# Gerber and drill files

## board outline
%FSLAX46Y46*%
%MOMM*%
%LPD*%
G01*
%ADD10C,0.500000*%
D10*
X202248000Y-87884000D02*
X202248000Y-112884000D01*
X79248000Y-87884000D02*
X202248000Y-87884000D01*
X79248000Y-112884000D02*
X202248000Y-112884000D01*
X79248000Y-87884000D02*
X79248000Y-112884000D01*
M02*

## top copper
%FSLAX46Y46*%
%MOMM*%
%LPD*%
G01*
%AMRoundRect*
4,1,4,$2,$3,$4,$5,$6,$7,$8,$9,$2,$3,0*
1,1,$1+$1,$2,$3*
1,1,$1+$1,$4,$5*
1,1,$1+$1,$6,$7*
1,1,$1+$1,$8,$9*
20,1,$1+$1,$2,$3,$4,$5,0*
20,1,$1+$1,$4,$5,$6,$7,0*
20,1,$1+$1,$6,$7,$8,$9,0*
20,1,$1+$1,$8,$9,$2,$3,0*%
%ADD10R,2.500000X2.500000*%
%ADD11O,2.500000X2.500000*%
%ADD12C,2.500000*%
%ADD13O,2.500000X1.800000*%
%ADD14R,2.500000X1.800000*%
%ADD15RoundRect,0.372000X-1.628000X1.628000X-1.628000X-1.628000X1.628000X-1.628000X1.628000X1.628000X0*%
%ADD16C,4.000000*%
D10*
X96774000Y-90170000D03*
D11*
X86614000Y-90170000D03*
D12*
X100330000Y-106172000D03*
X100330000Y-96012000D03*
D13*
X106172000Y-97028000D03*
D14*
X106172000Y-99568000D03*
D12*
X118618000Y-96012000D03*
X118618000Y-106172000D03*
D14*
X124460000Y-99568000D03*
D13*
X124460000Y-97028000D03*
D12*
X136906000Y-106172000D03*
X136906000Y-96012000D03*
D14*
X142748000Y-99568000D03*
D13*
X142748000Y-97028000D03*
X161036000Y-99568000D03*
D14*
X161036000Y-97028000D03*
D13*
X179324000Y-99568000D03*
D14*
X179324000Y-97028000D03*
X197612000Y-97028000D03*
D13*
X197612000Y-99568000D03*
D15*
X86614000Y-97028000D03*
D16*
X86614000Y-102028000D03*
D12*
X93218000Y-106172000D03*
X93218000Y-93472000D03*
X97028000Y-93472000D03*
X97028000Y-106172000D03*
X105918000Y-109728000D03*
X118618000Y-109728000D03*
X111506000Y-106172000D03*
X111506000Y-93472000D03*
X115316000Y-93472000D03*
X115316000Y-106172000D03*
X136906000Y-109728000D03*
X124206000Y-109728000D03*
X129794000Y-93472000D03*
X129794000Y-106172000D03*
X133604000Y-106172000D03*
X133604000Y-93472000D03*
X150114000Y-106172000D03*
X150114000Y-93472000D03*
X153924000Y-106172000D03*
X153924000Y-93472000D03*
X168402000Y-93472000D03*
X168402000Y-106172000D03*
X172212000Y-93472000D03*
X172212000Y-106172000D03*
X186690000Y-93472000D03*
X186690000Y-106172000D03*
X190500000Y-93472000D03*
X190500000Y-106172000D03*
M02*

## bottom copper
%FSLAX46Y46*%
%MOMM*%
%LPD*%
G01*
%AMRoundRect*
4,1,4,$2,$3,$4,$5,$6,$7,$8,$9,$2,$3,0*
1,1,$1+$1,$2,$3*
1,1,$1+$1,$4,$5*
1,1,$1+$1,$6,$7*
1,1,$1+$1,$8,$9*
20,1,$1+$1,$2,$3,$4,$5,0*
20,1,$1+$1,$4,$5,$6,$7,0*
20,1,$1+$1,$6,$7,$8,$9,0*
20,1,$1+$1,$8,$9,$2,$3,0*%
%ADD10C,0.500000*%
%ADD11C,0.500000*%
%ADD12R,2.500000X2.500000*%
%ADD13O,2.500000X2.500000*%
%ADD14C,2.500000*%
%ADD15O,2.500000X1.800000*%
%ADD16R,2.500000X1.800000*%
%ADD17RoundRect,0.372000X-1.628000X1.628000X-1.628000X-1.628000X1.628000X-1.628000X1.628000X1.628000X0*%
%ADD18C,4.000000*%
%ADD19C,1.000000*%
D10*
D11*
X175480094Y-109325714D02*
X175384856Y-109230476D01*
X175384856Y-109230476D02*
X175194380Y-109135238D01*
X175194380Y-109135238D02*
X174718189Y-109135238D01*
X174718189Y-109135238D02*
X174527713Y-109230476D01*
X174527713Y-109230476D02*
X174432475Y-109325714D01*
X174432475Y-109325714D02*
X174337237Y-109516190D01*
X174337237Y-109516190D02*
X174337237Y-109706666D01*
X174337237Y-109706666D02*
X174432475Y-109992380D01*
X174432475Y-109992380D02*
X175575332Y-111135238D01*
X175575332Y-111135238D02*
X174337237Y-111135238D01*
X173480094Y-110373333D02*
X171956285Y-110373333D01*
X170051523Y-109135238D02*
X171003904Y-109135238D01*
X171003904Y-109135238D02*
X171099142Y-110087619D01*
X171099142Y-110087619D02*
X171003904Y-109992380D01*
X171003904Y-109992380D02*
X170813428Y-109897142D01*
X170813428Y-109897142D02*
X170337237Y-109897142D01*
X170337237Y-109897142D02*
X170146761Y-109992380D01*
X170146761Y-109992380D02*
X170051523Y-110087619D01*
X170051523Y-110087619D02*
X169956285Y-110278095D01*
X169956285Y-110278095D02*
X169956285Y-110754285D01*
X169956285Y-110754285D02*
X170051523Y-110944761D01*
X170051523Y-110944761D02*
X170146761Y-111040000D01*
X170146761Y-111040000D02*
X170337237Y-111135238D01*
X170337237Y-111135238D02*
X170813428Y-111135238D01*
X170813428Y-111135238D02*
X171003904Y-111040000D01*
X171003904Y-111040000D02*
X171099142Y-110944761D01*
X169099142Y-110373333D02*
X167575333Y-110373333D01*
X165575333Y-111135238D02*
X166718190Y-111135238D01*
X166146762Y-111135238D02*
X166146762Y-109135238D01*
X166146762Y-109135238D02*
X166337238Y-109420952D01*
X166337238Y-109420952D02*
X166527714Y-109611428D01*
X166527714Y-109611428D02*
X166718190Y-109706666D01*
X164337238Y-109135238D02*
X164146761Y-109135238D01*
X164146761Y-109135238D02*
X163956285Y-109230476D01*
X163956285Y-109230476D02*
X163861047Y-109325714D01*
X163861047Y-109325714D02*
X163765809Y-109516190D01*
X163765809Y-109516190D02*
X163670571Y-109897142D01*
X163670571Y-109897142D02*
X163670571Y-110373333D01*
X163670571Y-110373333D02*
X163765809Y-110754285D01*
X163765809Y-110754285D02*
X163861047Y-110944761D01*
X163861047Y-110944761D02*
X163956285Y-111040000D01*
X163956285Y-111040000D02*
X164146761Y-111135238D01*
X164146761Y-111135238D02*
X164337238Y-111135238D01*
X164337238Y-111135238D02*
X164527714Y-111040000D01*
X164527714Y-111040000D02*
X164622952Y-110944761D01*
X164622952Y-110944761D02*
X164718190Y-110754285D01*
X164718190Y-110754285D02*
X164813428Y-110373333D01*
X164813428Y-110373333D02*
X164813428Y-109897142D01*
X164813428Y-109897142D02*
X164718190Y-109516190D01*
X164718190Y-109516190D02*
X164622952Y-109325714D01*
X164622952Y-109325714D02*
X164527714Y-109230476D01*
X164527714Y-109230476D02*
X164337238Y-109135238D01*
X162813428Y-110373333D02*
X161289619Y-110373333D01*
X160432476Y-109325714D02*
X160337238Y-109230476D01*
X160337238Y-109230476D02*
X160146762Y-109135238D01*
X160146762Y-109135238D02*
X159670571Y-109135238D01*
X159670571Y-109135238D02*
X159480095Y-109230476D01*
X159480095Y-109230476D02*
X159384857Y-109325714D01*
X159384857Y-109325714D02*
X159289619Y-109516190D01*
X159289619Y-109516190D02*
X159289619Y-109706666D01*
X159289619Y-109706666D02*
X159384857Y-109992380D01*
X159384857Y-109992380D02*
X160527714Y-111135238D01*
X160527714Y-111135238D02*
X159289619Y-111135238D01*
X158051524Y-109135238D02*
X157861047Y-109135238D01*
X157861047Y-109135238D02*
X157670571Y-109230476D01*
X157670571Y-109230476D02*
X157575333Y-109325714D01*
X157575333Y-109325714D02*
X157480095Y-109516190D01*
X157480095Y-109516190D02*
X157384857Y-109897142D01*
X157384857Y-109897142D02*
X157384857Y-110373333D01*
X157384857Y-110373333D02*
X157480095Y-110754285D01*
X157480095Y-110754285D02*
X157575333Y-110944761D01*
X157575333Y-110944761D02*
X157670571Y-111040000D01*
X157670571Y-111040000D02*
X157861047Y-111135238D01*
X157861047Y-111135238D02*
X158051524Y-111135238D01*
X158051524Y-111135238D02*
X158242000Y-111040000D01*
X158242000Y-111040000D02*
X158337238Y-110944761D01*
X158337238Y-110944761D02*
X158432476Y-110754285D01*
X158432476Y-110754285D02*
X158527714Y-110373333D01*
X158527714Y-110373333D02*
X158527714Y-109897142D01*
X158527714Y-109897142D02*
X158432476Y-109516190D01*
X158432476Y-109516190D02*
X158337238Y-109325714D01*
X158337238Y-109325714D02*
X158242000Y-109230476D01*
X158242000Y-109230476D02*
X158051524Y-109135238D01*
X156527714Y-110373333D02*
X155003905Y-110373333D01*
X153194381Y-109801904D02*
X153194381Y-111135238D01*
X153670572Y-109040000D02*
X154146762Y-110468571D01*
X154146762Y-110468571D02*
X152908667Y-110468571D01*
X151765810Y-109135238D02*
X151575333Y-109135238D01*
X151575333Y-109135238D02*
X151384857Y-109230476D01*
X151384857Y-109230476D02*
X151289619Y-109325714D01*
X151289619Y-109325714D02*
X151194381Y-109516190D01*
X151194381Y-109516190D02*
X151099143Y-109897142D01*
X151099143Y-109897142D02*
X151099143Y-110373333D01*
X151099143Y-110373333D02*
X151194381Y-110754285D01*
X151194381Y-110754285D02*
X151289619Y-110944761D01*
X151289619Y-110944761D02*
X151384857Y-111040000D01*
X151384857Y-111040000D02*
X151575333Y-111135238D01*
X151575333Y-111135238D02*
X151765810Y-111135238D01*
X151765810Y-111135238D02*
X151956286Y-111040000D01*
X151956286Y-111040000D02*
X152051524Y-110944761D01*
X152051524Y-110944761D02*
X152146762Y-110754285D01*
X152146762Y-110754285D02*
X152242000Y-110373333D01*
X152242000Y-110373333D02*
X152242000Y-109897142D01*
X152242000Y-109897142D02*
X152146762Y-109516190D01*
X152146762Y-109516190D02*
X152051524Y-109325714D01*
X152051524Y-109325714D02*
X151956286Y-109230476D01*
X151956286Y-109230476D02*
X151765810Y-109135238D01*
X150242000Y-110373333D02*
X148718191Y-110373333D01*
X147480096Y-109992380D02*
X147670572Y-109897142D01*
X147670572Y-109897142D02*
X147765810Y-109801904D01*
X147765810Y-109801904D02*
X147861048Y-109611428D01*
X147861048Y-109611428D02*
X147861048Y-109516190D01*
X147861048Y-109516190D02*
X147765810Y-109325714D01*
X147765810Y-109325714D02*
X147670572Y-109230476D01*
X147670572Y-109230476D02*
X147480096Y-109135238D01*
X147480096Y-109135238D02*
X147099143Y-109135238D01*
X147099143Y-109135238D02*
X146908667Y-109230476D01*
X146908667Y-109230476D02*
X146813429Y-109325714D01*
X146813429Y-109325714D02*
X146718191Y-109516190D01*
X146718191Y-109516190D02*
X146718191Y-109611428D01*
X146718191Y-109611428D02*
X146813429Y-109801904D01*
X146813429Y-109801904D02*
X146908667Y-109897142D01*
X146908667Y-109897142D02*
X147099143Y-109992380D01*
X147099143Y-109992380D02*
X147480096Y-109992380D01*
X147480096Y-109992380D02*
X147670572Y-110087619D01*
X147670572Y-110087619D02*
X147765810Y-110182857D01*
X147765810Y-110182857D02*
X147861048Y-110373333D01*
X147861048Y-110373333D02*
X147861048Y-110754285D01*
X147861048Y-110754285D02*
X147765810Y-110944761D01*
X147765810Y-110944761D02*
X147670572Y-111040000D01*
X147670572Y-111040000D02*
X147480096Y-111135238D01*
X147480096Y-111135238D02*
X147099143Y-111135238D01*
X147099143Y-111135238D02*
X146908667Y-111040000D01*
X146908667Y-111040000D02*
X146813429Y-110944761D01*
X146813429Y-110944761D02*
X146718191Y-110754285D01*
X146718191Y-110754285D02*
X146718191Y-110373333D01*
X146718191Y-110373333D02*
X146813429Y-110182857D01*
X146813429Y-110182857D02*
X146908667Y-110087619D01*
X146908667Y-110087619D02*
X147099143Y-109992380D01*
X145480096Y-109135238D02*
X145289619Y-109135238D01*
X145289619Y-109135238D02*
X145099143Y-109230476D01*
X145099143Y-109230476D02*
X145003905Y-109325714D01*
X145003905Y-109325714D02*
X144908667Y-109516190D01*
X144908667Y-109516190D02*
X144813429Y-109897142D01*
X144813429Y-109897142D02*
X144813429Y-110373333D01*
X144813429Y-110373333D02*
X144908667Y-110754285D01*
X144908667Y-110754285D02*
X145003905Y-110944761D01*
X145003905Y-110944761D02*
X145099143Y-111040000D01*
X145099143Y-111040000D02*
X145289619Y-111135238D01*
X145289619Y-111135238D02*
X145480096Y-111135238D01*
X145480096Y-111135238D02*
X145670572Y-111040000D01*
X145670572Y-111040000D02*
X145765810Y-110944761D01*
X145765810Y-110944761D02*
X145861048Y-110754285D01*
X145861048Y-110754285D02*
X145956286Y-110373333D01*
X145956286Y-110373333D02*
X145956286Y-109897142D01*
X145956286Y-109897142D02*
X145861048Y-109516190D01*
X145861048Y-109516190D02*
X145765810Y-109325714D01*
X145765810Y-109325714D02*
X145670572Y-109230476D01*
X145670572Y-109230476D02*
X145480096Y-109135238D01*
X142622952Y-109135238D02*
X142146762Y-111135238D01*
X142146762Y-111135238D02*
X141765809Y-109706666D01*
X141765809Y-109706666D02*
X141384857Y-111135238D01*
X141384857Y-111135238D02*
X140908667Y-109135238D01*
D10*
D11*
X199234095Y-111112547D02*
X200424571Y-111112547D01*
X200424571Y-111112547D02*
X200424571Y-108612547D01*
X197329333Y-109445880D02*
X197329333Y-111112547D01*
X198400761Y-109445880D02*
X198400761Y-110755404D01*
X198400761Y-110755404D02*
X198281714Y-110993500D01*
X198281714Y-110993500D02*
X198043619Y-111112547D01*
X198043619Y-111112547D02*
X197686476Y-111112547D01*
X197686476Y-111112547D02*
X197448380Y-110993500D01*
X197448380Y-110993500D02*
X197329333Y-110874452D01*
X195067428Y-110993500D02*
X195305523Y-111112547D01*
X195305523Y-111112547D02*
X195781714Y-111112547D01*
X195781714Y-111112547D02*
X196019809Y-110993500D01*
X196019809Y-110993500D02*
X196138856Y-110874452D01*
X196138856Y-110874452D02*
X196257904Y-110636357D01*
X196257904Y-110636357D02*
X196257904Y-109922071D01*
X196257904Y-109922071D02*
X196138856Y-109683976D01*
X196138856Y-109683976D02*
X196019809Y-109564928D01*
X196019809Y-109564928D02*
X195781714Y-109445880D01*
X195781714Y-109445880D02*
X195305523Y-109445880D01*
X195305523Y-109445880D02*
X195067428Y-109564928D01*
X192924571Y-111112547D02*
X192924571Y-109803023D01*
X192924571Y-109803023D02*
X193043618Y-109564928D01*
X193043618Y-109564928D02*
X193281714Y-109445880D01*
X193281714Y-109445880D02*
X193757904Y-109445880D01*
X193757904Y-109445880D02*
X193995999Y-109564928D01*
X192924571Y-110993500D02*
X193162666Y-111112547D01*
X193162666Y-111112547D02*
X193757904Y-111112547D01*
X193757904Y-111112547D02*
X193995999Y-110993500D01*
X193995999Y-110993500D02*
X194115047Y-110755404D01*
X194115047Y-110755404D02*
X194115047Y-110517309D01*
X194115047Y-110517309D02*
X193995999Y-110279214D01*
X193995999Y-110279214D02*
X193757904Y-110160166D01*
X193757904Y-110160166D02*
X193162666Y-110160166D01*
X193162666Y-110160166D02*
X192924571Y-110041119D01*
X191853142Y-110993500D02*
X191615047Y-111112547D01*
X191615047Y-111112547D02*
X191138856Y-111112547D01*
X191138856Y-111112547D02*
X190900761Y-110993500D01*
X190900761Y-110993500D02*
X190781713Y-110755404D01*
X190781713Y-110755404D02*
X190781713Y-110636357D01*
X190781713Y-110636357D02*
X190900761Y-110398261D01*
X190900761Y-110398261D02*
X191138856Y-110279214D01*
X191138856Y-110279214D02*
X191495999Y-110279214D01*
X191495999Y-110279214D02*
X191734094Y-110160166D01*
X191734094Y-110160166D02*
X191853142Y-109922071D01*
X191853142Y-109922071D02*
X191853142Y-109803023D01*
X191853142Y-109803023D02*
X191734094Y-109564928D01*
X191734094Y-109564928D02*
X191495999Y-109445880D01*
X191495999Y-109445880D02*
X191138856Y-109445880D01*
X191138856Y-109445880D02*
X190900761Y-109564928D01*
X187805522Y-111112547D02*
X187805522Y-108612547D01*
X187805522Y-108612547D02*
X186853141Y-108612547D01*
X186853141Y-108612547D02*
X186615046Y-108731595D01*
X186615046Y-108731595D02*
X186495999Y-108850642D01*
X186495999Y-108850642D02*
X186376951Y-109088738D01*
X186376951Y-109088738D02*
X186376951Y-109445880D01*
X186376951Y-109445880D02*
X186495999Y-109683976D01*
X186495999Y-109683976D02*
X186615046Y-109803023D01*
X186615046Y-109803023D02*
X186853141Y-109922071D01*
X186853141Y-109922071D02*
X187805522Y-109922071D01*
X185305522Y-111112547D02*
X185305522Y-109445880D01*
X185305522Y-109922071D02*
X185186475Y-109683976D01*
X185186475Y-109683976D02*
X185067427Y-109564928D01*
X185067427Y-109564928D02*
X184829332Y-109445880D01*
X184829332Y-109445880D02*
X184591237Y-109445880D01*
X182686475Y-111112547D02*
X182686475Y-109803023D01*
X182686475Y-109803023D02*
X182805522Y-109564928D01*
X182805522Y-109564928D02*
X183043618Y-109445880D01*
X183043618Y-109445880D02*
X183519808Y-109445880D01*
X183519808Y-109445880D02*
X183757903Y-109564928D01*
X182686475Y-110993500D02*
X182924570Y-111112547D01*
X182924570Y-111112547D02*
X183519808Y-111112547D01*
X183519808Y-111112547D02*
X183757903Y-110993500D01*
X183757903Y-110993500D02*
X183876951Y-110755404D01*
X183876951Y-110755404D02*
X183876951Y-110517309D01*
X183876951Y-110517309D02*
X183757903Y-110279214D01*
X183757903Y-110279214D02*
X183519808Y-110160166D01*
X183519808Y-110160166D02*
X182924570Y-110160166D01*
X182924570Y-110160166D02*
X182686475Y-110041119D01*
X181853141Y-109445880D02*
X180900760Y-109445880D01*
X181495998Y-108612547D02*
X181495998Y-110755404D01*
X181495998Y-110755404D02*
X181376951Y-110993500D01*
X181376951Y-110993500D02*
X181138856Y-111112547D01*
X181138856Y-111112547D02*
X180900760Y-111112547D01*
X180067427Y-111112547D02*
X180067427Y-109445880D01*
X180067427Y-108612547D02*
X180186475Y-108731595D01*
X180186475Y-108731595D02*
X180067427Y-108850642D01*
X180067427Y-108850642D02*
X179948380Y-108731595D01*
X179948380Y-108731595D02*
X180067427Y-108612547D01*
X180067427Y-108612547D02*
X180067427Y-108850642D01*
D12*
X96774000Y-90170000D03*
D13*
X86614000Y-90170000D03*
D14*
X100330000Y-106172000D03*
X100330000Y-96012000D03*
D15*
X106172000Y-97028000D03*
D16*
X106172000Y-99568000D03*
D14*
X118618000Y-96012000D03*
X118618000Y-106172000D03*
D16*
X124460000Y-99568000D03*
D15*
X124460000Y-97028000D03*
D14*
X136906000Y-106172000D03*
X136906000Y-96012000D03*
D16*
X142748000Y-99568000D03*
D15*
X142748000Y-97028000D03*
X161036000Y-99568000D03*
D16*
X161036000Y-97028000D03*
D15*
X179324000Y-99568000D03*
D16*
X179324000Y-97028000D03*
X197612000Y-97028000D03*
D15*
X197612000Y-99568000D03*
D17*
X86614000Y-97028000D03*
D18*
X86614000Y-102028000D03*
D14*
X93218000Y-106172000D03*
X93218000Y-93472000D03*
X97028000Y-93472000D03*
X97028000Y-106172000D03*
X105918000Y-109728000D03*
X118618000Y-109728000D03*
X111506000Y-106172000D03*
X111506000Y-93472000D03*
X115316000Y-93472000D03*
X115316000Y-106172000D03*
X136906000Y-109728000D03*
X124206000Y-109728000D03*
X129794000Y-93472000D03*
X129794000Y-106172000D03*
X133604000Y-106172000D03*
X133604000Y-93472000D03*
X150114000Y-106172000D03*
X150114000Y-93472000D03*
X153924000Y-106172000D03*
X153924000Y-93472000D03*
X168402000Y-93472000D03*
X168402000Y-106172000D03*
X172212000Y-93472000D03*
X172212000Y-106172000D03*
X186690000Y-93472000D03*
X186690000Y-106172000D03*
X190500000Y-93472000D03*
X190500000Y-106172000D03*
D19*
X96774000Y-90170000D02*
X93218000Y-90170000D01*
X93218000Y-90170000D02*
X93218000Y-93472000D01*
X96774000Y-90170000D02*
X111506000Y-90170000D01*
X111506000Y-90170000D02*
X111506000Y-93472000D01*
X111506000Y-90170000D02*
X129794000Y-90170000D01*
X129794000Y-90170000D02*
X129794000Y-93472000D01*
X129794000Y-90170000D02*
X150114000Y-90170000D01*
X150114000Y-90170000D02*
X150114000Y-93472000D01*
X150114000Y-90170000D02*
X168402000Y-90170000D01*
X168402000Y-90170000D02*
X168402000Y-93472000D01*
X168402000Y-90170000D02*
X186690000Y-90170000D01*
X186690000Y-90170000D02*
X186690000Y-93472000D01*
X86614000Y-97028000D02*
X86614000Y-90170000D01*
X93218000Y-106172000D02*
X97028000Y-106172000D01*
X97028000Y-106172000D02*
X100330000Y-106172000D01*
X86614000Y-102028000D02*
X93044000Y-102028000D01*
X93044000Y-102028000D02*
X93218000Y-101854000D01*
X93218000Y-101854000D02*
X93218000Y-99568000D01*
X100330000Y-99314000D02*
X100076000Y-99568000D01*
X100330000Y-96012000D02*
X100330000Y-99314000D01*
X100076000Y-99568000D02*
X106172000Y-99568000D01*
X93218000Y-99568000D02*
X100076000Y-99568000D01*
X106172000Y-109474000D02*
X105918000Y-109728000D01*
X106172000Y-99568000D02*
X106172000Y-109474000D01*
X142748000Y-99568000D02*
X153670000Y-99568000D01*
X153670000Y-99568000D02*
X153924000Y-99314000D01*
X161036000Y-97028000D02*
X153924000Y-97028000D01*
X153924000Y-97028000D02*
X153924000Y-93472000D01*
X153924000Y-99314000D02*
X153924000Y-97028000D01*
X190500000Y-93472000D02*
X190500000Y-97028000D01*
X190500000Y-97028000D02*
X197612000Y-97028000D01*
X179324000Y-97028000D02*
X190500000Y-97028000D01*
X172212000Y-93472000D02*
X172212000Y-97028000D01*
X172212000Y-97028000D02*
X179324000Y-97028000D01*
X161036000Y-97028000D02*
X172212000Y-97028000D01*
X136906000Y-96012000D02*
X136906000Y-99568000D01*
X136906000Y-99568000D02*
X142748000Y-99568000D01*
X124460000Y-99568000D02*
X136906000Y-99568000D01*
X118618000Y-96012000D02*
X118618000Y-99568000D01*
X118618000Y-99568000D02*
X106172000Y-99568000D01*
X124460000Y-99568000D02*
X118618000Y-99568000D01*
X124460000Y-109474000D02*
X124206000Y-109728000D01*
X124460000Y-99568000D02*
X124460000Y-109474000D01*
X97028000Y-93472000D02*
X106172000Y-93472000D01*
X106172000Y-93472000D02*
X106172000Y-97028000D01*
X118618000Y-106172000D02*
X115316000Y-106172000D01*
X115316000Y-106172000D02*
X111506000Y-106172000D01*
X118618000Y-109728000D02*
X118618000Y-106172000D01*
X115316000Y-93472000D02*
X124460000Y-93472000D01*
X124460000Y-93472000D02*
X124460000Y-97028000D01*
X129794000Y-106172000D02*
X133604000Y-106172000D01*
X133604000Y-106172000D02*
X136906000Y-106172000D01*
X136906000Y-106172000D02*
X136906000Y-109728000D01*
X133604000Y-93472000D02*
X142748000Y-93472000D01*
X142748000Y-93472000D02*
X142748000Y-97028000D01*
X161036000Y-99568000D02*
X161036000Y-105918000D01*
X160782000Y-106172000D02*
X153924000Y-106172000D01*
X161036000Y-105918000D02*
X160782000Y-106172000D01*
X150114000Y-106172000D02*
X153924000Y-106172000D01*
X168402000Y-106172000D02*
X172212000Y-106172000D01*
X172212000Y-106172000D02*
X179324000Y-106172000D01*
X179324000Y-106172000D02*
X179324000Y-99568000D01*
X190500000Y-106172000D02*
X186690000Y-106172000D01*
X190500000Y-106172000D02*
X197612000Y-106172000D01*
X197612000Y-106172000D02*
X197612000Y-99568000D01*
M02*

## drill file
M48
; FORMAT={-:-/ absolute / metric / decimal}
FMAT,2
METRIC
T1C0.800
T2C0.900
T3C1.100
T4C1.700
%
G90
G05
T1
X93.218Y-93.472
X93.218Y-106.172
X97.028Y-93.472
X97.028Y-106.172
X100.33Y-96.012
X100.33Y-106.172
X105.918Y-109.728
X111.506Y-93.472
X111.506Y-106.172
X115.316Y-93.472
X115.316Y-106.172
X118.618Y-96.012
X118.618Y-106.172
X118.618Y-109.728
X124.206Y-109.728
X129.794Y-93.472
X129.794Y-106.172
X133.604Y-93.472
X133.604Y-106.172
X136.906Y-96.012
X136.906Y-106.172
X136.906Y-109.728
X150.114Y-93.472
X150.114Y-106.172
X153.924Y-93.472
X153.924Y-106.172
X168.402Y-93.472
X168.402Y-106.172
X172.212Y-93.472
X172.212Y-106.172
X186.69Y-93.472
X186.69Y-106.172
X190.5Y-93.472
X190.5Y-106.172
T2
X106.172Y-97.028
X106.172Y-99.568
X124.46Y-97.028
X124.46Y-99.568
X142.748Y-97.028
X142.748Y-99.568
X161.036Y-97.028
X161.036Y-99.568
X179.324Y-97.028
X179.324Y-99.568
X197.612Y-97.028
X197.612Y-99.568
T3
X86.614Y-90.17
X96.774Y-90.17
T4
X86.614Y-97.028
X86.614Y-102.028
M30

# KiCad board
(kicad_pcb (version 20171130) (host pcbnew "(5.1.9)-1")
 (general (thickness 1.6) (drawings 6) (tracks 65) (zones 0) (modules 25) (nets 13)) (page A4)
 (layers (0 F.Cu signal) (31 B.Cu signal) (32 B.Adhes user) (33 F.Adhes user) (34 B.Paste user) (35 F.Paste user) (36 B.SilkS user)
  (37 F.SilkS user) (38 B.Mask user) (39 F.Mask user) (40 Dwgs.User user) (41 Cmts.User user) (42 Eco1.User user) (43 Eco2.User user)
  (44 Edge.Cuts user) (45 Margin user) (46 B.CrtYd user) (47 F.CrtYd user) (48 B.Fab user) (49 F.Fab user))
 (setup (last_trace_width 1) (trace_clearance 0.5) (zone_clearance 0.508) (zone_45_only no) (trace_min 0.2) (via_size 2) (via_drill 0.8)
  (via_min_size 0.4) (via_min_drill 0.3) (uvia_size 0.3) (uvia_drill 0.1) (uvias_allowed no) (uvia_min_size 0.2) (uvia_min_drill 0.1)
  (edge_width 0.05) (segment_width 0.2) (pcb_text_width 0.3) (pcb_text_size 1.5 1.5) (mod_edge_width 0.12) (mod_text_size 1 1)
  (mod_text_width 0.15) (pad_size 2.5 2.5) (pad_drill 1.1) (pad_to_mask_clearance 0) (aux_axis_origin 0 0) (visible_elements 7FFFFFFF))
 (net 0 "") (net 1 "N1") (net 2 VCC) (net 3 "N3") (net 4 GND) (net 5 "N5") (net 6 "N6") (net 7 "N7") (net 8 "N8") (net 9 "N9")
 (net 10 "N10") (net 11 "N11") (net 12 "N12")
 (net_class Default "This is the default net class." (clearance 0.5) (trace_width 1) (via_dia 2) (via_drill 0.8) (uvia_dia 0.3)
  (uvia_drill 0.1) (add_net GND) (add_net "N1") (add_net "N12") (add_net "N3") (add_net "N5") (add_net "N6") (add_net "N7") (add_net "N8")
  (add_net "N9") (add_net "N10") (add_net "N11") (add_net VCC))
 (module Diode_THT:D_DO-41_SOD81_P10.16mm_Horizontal (layer F.Cu) (at 96.774 90.17 180)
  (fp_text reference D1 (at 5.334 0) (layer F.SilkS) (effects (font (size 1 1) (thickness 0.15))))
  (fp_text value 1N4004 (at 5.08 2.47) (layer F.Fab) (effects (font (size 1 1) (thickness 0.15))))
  (pad 1 thru_hole rect (at 0 0 180) (size 2.5 2.5) (drill 1.1) (layers *.Cu *.Mask) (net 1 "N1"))
  (pad 2 thru_hole oval (at 10.16 0 180) (size 2.5 2.5) (drill 1.1) (layers *.Cu *.Mask) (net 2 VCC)))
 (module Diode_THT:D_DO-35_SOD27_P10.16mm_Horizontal (layer F.Cu) (at 100.33 106.172 90)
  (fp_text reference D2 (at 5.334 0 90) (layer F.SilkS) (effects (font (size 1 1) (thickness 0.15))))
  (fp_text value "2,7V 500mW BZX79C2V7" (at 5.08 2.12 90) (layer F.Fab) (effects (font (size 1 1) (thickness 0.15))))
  (pad 1 thru_hole circle (at 0 0 90) (size 2.5 2.5) (drill 0.8) (layers *.Cu *.Mask) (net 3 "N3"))
  (pad 2 thru_hole circle (at 10.16 0 90) (size 2.5 2.5) (drill 0.8) (layers *.Cu *.Mask) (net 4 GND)))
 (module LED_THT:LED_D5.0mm (layer F.Cu) (at 106.172 99.568 90)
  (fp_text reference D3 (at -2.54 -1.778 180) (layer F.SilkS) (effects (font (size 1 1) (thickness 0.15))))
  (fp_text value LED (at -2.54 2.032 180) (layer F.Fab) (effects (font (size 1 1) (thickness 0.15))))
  (pad 2 thru_hole oval (at 2.54 0 90) (size 1.8 2.5) (drill 0.9) (layers *.Cu *.Mask) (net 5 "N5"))
  (pad 1 thru_hole rect (at 0 0 90) (size 1.8 2.5) (drill 0.9) (layers *.Cu *.Mask) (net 4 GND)))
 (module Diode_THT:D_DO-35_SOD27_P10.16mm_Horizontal (layer F.Cu) (at 118.618 106.172 90)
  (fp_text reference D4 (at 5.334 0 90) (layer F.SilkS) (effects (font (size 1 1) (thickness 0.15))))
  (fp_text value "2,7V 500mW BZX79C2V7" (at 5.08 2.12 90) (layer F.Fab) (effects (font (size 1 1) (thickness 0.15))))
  (pad 2 thru_hole circle (at 10.16 0 90) (size 2.5 2.5) (drill 0.8) (layers *.Cu *.Mask) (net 4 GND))
  (pad 1 thru_hole circle (at 0 0 90) (size 2.5 2.5) (drill 0.8) (layers *.Cu *.Mask) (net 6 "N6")))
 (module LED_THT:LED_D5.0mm (layer F.Cu) (at 124.46 99.568 90)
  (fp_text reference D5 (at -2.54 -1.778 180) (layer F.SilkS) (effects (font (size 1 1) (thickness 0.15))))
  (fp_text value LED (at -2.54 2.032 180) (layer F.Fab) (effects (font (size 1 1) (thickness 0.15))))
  (pad 1 thru_hole rect (at 0 0 90) (size 1.8 2.5) (drill 0.9) (layers *.Cu *.Mask) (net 4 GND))
  (pad 2 thru_hole oval (at 2.54 0 90) (size 1.8 2.5) (drill 0.9) (layers *.Cu *.Mask) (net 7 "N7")))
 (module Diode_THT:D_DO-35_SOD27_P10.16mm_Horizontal (layer F.Cu) (at 136.906 106.172 90)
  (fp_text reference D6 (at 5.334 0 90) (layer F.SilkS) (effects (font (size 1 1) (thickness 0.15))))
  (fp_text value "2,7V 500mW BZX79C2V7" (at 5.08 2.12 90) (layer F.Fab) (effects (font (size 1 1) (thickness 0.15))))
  (pad 1 thru_hole circle (at 0 0 90) (size 2.5 2.5) (drill 0.8) (layers *.Cu *.Mask) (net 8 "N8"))
  (pad 2 thru_hole circle (at 10.16 0 90) (size 2.5 2.5) (drill 0.8) (layers *.Cu *.Mask) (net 4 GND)))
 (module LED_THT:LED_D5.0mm (layer F.Cu) (at 142.748 99.568 90)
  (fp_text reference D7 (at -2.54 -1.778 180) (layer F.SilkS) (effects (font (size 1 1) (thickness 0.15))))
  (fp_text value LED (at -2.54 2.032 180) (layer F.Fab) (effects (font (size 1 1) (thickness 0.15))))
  (pad 1 thru_hole rect (at 0 0 90) (size 1.8 2.5) (drill 0.9) (layers *.Cu *.Mask) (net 4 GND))
  (pad 2 thru_hole oval (at 2.54 0 90) (size 1.8 2.5) (drill 0.9) (layers *.Cu *.Mask) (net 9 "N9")))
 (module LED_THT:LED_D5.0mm (layer F.Cu) (at 161.036 97.028 270)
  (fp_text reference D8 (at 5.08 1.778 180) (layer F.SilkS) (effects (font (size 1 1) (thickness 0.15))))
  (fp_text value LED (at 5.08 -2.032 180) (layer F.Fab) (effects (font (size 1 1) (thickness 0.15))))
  (pad 2 thru_hole oval (at 2.54 0 270) (size 1.8 2.5) (drill 0.9) (layers *.Cu *.Mask) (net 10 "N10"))
  (pad 1 thru_hole rect (at 0 0 270) (size 1.8 2.5) (drill 0.9) (layers *.Cu *.Mask) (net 4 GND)))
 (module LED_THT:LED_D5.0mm (layer F.Cu) (at 179.324 97.028 270)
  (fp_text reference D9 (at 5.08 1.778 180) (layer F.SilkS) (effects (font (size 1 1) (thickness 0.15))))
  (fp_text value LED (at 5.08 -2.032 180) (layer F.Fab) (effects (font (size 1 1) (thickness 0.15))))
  (pad 2 thru_hole oval (at 2.54 0 270) (size 1.8 2.5) (drill 0.9) (layers *.Cu *.Mask) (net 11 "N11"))
  (pad 1 thru_hole rect (at 0 0 270) (size 1.8 2.5) (drill 0.9) (layers *.Cu *.Mask) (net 4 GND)))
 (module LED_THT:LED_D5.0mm (layer F.Cu) (at 197.612 97.028 270)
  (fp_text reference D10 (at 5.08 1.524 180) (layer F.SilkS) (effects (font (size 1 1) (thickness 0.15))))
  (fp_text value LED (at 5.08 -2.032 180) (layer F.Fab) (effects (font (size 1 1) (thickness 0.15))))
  (pad 1 thru_hole rect (at 0 0 270) (size 1.8 2.5) (drill 0.9) (layers *.Cu *.Mask) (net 4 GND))
  (pad 2 thru_hole oval (at 2.54 0 270) (size 1.8 2.5) (drill 0.9) (layers *.Cu *.Mask) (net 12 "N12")))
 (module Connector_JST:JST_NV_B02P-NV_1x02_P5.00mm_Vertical (layer F.Cu) (at 86.614 97.028 270)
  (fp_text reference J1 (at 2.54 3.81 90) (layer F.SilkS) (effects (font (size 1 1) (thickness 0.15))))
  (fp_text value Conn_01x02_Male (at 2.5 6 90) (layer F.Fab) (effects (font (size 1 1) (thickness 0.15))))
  (pad 1 thru_hole roundrect (at 0 0 270) (size 4 4) (drill 1.7) (layers *.Cu *.Mask) (roundrect_rratio 0.09300000000000001) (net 2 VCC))
  (pad 2 thru_hole circle (at 5 0 270) (size 4 4) (drill 1.7) (layers *.Cu *.Mask) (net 4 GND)))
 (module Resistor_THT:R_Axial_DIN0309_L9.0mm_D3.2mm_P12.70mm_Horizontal (layer F.Cu) (at 93.218 93.472 270)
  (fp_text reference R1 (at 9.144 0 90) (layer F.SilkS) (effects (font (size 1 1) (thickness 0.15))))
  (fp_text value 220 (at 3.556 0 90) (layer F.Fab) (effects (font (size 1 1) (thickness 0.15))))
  (pad 2 thru_hole circle (at 12.7 0 270) (size 2.5 2.5) (drill 0.8) (layers *.Cu *.Mask) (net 3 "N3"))
  (pad 1 thru_hole circle (at 0 0 270) (size 2.5 2.5) (drill 0.8) (layers *.Cu *.Mask) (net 1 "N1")))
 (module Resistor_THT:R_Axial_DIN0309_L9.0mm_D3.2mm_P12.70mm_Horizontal (layer F.Cu) (at 97.028 93.472 270)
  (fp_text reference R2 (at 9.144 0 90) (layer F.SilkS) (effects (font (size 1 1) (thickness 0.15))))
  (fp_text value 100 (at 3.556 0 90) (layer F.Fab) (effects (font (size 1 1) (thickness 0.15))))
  (pad 1 thru_hole circle (at 0 0 270) (size 2.5 2.5) (drill 0.8) (layers *.Cu *.Mask) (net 5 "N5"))
  (pad 2 thru_hole circle (at 12.7 0 270) (size 2.5 2.5) (drill 0.8) (layers *.Cu *.Mask) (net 3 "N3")))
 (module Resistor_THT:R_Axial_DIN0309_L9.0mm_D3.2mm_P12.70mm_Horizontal (layer F.Cu) (at 118.618 109.728 180)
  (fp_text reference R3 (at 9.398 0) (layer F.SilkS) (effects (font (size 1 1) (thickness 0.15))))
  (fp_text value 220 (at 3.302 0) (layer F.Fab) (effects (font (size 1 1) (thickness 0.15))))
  (pad 2 thru_hole circle (at 12.7 0 180) (size 2.5 2.5) (drill 0.8) (layers *.Cu *.Mask) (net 4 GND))
  (pad 1 thru_hole circle (at 0 0 180) (size 2.5 2.5) (drill 0.8) (layers *.Cu *.Mask) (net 6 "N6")))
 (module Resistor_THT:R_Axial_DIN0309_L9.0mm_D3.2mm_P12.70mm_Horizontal (layer F.Cu) (at 111.506 93.472 270)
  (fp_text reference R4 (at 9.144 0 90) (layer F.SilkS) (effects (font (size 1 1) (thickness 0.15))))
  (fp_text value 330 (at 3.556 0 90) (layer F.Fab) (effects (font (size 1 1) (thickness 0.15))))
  (pad 2 thru_hole circle (at 12.7 0 270) (size 2.5 2.5) (drill 0.8) (layers *.Cu *.Mask) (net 6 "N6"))
  (pad 1 thru_hole circle (at 0 0 270) (size 2.5 2.5) (drill 0.8) (layers *.Cu *.Mask) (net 1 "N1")))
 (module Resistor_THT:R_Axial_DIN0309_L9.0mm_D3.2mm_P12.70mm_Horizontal (layer F.Cu) (at 115.316 93.472 270)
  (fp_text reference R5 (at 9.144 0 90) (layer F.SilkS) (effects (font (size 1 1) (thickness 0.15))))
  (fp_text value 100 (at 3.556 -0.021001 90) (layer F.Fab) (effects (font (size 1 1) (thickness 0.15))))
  (pad 1 thru_hole circle (at 0 0 270) (size 2.5 2.5) (drill 0.8) (layers *.Cu *.Mask) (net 7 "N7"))
  (pad 2 thru_hole circle (at 12.7 0 270) (size 2.5 2.5) (drill 0.8) (layers *.Cu *.Mask) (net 6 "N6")))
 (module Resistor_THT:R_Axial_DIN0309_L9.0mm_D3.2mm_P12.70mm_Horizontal (layer F.Cu) (at 136.906 109.728 180)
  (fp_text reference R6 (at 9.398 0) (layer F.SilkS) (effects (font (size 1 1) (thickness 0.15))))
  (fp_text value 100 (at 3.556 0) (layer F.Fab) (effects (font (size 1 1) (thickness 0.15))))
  (pad 1 thru_hole circle (at 0 0 180) (size 2.5 2.5) (drill 0.8) (layers *.Cu *.Mask) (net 8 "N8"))
  (pad 2 thru_hole circle (at 12.7 0 180) (size 2.5 2.5) (drill 0.8) (layers *.Cu *.Mask) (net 4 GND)))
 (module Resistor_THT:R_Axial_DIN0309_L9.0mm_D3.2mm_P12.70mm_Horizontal (layer F.Cu) (at 129.794 93.472 270)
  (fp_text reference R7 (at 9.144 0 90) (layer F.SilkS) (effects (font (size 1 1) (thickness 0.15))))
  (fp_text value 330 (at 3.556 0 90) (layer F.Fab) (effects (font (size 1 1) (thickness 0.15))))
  (pad 1 thru_hole circle (at 0 0 270) (size 2.5 2.5) (drill 0.8) (layers *.Cu *.Mask) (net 1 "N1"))
  (pad 2 thru_hole circle (at 12.7 0 270) (size 2.5 2.5) (drill 0.8) (layers *.Cu *.Mask) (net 8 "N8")))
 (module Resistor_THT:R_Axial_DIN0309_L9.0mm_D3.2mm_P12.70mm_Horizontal (layer F.Cu) (at 133.604 93.472 270)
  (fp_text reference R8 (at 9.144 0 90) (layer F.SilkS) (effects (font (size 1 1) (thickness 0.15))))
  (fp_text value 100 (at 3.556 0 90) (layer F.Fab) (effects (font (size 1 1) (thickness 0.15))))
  (pad 2 thru_hole circle (at 12.7 0 270) (size 2.5 2.5) (drill 0.8) (layers *.Cu *.Mask) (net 8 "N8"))
  (pad 1 thru_hole circle (at 0 0 270) (size 2.5 2.5) (drill 0.8) (layers *.Cu *.Mask) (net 9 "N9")))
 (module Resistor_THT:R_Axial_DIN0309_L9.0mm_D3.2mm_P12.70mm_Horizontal (layer F.Cu) (at 150.114 93.472 270)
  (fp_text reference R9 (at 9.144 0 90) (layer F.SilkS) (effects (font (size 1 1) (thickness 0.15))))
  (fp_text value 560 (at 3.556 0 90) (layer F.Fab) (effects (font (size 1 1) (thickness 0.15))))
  (pad 2 thru_hole circle (at 12.7 0 270) (size 2.5 2.5) (drill 0.8) (layers *.Cu *.Mask) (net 10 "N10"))
  (pad 1 thru_hole circle (at 0 0 270) (size 2.5 2.5) (drill 0.8) (layers *.Cu *.Mask) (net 1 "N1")))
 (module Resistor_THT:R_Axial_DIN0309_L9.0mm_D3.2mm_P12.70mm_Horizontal (layer F.Cu) (at 153.924 106.172 90)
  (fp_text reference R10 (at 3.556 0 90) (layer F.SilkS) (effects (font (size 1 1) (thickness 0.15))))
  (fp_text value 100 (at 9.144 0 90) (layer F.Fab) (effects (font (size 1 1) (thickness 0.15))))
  (pad 1 thru_hole circle (at 0 0 90) (size 2.5 2.5) (drill 0.8) (layers *.Cu *.Mask) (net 10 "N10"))
  (pad 2 thru_hole circle (at 12.7 0 90) (size 2.5 2.5) (drill 0.8) (layers *.Cu *.Mask) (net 4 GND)))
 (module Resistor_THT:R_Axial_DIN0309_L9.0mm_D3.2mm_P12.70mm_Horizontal (layer F.Cu) (at 168.402 93.472 270)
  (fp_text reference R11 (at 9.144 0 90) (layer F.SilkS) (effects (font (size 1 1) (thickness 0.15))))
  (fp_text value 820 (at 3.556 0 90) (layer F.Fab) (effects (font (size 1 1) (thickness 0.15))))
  (pad 1 thru_hole circle (at 0 0 270) (size 2.5 2.5) (drill 0.8) (layers *.Cu *.Mask) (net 1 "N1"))
  (pad 2 thru_hole circle (at 12.7 0 270) (size 2.5 2.5) (drill 0.8) (layers *.Cu *.Mask) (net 11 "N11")))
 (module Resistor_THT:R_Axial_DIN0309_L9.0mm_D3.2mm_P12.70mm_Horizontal (layer F.Cu) (at 172.212 106.172 90)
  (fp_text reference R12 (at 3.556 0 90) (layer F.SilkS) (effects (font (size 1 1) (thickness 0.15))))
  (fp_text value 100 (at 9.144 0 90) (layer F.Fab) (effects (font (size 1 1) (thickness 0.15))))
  (pad 2 thru_hole circle (at 12.7 0 90) (size 2.5 2.5) (drill 0.8) (layers *.Cu *.Mask) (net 4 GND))
  (pad 1 thru_hole circle (at 0 0 90) (size 2.5 2.5) (drill 0.8) (layers *.Cu *.Mask) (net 11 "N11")))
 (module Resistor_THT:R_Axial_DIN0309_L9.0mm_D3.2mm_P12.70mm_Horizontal (layer F.Cu) (at 186.69 93.472 270)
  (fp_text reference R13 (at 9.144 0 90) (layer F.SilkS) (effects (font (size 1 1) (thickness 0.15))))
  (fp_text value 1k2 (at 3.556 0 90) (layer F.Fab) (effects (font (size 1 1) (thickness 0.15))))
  (pad 1 thru_hole circle (at 0 0 270) (size 2.5 2.5) (drill 0.8) (layers *.Cu *.Mask) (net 1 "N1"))
  (pad 2 thru_hole circle (at 12.7 0 270) (size 2.5 2.5) (drill 0.8) (layers *.Cu *.Mask) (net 12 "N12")))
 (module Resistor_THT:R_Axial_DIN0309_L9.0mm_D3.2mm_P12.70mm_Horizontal (layer F.Cu) (at 190.5 106.172 90)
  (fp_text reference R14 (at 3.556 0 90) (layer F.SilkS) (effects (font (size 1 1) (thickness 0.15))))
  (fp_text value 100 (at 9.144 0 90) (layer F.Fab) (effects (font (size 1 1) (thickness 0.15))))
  (pad 2 thru_hole circle (at 12.7 0 90) (size 2.5 2.5) (drill 0.8) (layers *.Cu *.Mask) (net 4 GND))
  (pad 1 thru_hole circle (at 0 0 90) (size 2.5 2.5) (drill 0.8) (layers *.Cu *.Mask) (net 12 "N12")))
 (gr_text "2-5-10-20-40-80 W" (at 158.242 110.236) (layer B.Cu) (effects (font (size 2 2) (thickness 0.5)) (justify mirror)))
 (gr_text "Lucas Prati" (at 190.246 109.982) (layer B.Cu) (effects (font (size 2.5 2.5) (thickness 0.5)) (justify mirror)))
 (gr_line (start 202.248 87.884) (end 202.248 112.884) (layer Edge.Cuts) (width 0.5))
 (gr_line (start 79.248 87.884) (end 202.248 87.884) (layer Edge.Cuts) (width 0.5))
 (gr_line (start 79.248 112.884) (end 202.248 112.884) (layer Edge.Cuts) (width 0.5))
 (gr_line (start 79.248 87.884) (end 79.248 112.884) (layer Edge.Cuts) (width 0.5))
 (segment (start 96.774 90.17) (end 93.218 90.17) (width 1) (layer B.Cu) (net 1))
 (segment (start 93.218 90.17) (end 93.218 93.472) (width 1) (layer B.Cu) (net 1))
 (segment (start 96.774 90.17) (end 111.506 90.17) (width 1) (layer B.Cu) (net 1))
 (segment (start 111.506 90.17) (end 111.506 93.472) (width 1) (layer B.Cu) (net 1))
 (segment (start 111.506 90.17) (end 129.794 90.17) (width 1) (layer B.Cu) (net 1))
 (segment (start 129.794 90.17) (end 129.794 93.472) (width 1) (layer B.Cu) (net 1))
 (segment (start 129.794 90.17) (end 150.114 90.17) (width 1) (layer B.Cu) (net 1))
 (segment (start 150.114 90.17) (end 150.114 93.472) (width 1) (layer B.Cu) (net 1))
 (segment (start 150.114 90.17) (end 168.402 90.17) (width 1) (layer B.Cu) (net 1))
 (segment (start 168.402 90.17) (end 168.402 93.472) (width 1) (layer B.Cu) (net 1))
 (segment (start 168.402 90.17) (end 186.69 90.17) (width 1) (layer B.Cu) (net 1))
 (segment (start 186.69 90.17) (end 186.69 93.472) (width 1) (layer B.Cu) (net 1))
 (segment (start 86.614 97.028) (end 86.614 90.17) (width 1) (layer B.Cu) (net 2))
 (segment (start 93.218 106.172) (end 97.028 106.172) (width 1) (layer B.Cu) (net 3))
 (segment (start 97.028 106.172) (end 100.33 106.172) (width 1) (layer B.Cu) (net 3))
 (segment (start 86.614 102.028) (end 93.044 102.028) (width 1) (layer B.Cu) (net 4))
 (segment (start 93.044 102.028) (end 93.218 101.854) (width 1) (layer B.Cu) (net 4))
 (segment (start 93.218 101.854) (end 93.218 99.568) (width 1) (layer B.Cu) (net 4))
 (segment (start 100.33 99.314) (end 100.076 99.568) (width 1) (layer B.Cu) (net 4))
 (segment (start 100.33 96.012) (end 100.33 99.314) (width 1) (layer B.Cu) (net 4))
 (segment (start 100.076 99.568) (end 106.172 99.568) (width 1) (layer B.Cu) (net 4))
 (segment (start 93.218 99.568) (end 100.076 99.568) (width 1) (layer B.Cu) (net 4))
 (segment (start 106.172 109.474) (end 105.918 109.728) (width 1) (layer B.Cu) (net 4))
 (segment (start 106.172 99.568) (end 106.172 109.474) (width 1) (layer B.Cu) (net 4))
 (segment (start 142.748 99.568) (end 153.67 99.568) (width 1) (layer B.Cu) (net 4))
 (segment (start 153.67 99.568) (end 153.924 99.314) (width 1) (layer B.Cu) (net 4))
 (segment (start 161.036 97.028) (end 153.924 97.028) (width 1) (layer B.Cu) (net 4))
 (segment (start 153.924 97.028) (end 153.924 93.472) (width 1) (layer B.Cu) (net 4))
 (segment (start 153.924 99.314) (end 153.924 97.028) (width 1) (layer B.Cu) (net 4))
 (segment (start 190.5 93.472) (end 190.5 97.028) (width 1) (layer B.Cu) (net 4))
 (segment (start 190.5 97.028) (end 197.612 97.028) (width 1) (layer B.Cu) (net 4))
 (segment (start 179.324 97.028) (end 190.5 97.028) (width 1) (layer B.Cu) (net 4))
 (segment (start 172.212 93.472) (end 172.212 97.028) (width 1) (layer B.Cu) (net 4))
 (segment (start 172.212 97.028) (end 179.324 97.028) (width 1) (layer B.Cu) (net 4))
 (segment (start 161.036 97.028) (end 172.212 97.028) (width 1) (layer B.Cu) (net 4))
 (segment (start 136.906 96.012) (end 136.906 99.568) (width 1) (layer B.Cu) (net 4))
 (segment (start 136.906 99.568) (end 142.748 99.568) (width 1) (layer B.Cu) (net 4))
 (segment (start 124.46 99.568) (end 136.906 99.568) (width 1) (layer B.Cu) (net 4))
 (segment (start 118.618 96.012) (end 118.618 99.568) (width 1) (layer B.Cu) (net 4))
 (segment (start 118.618 99.568) (end 106.172 99.568) (width 1) (layer B.Cu) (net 4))
 (segment (start 124.46 99.568) (end 118.618 99.568) (width 1) (layer B.Cu) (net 4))
 (segment (start 124.46 109.474) (end 124.206 109.728) (width 1) (layer B.Cu) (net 4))
 (segment (start 124.46 99.568) (end 124.46 109.474) (width 1) (layer B.Cu) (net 4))
 (segment (start 97.028 93.472) (end 106.172 93.472) (width 1) (layer B.Cu) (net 5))
 (segment (start 106.172 93.472) (end 106.172 97.028) (width 1) (layer B.Cu) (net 5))
 (segment (start 118.618 106.172) (end 115.316 106.172) (width 1) (layer B.Cu) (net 6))
 (segment (start 115.316 106.172) (end 111.506 106.172) (width 1) (layer B.Cu) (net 6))
 (segment (start 118.618 109.728) (end 118.618 106.172) (width 1) (layer B.Cu) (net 6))
 (segment (start 115.316 93.472) (end 124.46 93.472) (width 1) (layer B.Cu) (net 7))
 (segment (start 124.46 93.472) (end 124.46 97.028) (width 1) (layer B.Cu) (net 7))
 (segment (start 129.794 106.172) (end 133.604 106.172) (width 1) (layer B.Cu) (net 8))
 (segment (start 133.604 106.172) (end 136.906 106.172) (width 1) (layer B.Cu) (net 8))
 (segment (start 136.906 106.172) (end 136.906 109.728) (width 1) (layer B.Cu) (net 8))
 (segment (start 133.604 93.472) (end 142.748 93.472) (width 1) (layer B.Cu) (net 9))
 (segment (start 142.748 93.472) (end 142.748 97.028) (width 1) (layer B.Cu) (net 9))
 (segment (start 161.036 99.568) (end 161.036 105.918) (width 1) (layer B.Cu) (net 10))
 (segment (start 160.782 106.172) (end 153.924 106.172) (width 1) (layer B.Cu) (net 10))
 (segment (start 161.036 105.918) (end 160.782 106.172) (width 1) (layer B.Cu) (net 10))
 (segment (start 150.114 106.172) (end 153.924 106.172) (width 1) (layer B.Cu) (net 10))
 (segment (start 168.402 106.172) (end 172.212 106.172) (width 1) (layer B.Cu) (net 11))
 (segment (start 172.212 106.172) (end 179.324 106.172) (width 1) (layer B.Cu) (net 11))
 (segment (start 179.324 106.172) (end 179.324 99.568) (width 1) (layer B.Cu) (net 11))
 (segment (start 190.5 106.172) (end 186.69 106.172) (width 1) (layer B.Cu) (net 12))
 (segment (start 190.5 106.172) (end 197.612 106.172) (width 1) (layer B.Cu) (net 12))
 (segment (start 197.612 106.172) (end 197.612 99.568) (width 1) (layer B.Cu) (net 12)))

